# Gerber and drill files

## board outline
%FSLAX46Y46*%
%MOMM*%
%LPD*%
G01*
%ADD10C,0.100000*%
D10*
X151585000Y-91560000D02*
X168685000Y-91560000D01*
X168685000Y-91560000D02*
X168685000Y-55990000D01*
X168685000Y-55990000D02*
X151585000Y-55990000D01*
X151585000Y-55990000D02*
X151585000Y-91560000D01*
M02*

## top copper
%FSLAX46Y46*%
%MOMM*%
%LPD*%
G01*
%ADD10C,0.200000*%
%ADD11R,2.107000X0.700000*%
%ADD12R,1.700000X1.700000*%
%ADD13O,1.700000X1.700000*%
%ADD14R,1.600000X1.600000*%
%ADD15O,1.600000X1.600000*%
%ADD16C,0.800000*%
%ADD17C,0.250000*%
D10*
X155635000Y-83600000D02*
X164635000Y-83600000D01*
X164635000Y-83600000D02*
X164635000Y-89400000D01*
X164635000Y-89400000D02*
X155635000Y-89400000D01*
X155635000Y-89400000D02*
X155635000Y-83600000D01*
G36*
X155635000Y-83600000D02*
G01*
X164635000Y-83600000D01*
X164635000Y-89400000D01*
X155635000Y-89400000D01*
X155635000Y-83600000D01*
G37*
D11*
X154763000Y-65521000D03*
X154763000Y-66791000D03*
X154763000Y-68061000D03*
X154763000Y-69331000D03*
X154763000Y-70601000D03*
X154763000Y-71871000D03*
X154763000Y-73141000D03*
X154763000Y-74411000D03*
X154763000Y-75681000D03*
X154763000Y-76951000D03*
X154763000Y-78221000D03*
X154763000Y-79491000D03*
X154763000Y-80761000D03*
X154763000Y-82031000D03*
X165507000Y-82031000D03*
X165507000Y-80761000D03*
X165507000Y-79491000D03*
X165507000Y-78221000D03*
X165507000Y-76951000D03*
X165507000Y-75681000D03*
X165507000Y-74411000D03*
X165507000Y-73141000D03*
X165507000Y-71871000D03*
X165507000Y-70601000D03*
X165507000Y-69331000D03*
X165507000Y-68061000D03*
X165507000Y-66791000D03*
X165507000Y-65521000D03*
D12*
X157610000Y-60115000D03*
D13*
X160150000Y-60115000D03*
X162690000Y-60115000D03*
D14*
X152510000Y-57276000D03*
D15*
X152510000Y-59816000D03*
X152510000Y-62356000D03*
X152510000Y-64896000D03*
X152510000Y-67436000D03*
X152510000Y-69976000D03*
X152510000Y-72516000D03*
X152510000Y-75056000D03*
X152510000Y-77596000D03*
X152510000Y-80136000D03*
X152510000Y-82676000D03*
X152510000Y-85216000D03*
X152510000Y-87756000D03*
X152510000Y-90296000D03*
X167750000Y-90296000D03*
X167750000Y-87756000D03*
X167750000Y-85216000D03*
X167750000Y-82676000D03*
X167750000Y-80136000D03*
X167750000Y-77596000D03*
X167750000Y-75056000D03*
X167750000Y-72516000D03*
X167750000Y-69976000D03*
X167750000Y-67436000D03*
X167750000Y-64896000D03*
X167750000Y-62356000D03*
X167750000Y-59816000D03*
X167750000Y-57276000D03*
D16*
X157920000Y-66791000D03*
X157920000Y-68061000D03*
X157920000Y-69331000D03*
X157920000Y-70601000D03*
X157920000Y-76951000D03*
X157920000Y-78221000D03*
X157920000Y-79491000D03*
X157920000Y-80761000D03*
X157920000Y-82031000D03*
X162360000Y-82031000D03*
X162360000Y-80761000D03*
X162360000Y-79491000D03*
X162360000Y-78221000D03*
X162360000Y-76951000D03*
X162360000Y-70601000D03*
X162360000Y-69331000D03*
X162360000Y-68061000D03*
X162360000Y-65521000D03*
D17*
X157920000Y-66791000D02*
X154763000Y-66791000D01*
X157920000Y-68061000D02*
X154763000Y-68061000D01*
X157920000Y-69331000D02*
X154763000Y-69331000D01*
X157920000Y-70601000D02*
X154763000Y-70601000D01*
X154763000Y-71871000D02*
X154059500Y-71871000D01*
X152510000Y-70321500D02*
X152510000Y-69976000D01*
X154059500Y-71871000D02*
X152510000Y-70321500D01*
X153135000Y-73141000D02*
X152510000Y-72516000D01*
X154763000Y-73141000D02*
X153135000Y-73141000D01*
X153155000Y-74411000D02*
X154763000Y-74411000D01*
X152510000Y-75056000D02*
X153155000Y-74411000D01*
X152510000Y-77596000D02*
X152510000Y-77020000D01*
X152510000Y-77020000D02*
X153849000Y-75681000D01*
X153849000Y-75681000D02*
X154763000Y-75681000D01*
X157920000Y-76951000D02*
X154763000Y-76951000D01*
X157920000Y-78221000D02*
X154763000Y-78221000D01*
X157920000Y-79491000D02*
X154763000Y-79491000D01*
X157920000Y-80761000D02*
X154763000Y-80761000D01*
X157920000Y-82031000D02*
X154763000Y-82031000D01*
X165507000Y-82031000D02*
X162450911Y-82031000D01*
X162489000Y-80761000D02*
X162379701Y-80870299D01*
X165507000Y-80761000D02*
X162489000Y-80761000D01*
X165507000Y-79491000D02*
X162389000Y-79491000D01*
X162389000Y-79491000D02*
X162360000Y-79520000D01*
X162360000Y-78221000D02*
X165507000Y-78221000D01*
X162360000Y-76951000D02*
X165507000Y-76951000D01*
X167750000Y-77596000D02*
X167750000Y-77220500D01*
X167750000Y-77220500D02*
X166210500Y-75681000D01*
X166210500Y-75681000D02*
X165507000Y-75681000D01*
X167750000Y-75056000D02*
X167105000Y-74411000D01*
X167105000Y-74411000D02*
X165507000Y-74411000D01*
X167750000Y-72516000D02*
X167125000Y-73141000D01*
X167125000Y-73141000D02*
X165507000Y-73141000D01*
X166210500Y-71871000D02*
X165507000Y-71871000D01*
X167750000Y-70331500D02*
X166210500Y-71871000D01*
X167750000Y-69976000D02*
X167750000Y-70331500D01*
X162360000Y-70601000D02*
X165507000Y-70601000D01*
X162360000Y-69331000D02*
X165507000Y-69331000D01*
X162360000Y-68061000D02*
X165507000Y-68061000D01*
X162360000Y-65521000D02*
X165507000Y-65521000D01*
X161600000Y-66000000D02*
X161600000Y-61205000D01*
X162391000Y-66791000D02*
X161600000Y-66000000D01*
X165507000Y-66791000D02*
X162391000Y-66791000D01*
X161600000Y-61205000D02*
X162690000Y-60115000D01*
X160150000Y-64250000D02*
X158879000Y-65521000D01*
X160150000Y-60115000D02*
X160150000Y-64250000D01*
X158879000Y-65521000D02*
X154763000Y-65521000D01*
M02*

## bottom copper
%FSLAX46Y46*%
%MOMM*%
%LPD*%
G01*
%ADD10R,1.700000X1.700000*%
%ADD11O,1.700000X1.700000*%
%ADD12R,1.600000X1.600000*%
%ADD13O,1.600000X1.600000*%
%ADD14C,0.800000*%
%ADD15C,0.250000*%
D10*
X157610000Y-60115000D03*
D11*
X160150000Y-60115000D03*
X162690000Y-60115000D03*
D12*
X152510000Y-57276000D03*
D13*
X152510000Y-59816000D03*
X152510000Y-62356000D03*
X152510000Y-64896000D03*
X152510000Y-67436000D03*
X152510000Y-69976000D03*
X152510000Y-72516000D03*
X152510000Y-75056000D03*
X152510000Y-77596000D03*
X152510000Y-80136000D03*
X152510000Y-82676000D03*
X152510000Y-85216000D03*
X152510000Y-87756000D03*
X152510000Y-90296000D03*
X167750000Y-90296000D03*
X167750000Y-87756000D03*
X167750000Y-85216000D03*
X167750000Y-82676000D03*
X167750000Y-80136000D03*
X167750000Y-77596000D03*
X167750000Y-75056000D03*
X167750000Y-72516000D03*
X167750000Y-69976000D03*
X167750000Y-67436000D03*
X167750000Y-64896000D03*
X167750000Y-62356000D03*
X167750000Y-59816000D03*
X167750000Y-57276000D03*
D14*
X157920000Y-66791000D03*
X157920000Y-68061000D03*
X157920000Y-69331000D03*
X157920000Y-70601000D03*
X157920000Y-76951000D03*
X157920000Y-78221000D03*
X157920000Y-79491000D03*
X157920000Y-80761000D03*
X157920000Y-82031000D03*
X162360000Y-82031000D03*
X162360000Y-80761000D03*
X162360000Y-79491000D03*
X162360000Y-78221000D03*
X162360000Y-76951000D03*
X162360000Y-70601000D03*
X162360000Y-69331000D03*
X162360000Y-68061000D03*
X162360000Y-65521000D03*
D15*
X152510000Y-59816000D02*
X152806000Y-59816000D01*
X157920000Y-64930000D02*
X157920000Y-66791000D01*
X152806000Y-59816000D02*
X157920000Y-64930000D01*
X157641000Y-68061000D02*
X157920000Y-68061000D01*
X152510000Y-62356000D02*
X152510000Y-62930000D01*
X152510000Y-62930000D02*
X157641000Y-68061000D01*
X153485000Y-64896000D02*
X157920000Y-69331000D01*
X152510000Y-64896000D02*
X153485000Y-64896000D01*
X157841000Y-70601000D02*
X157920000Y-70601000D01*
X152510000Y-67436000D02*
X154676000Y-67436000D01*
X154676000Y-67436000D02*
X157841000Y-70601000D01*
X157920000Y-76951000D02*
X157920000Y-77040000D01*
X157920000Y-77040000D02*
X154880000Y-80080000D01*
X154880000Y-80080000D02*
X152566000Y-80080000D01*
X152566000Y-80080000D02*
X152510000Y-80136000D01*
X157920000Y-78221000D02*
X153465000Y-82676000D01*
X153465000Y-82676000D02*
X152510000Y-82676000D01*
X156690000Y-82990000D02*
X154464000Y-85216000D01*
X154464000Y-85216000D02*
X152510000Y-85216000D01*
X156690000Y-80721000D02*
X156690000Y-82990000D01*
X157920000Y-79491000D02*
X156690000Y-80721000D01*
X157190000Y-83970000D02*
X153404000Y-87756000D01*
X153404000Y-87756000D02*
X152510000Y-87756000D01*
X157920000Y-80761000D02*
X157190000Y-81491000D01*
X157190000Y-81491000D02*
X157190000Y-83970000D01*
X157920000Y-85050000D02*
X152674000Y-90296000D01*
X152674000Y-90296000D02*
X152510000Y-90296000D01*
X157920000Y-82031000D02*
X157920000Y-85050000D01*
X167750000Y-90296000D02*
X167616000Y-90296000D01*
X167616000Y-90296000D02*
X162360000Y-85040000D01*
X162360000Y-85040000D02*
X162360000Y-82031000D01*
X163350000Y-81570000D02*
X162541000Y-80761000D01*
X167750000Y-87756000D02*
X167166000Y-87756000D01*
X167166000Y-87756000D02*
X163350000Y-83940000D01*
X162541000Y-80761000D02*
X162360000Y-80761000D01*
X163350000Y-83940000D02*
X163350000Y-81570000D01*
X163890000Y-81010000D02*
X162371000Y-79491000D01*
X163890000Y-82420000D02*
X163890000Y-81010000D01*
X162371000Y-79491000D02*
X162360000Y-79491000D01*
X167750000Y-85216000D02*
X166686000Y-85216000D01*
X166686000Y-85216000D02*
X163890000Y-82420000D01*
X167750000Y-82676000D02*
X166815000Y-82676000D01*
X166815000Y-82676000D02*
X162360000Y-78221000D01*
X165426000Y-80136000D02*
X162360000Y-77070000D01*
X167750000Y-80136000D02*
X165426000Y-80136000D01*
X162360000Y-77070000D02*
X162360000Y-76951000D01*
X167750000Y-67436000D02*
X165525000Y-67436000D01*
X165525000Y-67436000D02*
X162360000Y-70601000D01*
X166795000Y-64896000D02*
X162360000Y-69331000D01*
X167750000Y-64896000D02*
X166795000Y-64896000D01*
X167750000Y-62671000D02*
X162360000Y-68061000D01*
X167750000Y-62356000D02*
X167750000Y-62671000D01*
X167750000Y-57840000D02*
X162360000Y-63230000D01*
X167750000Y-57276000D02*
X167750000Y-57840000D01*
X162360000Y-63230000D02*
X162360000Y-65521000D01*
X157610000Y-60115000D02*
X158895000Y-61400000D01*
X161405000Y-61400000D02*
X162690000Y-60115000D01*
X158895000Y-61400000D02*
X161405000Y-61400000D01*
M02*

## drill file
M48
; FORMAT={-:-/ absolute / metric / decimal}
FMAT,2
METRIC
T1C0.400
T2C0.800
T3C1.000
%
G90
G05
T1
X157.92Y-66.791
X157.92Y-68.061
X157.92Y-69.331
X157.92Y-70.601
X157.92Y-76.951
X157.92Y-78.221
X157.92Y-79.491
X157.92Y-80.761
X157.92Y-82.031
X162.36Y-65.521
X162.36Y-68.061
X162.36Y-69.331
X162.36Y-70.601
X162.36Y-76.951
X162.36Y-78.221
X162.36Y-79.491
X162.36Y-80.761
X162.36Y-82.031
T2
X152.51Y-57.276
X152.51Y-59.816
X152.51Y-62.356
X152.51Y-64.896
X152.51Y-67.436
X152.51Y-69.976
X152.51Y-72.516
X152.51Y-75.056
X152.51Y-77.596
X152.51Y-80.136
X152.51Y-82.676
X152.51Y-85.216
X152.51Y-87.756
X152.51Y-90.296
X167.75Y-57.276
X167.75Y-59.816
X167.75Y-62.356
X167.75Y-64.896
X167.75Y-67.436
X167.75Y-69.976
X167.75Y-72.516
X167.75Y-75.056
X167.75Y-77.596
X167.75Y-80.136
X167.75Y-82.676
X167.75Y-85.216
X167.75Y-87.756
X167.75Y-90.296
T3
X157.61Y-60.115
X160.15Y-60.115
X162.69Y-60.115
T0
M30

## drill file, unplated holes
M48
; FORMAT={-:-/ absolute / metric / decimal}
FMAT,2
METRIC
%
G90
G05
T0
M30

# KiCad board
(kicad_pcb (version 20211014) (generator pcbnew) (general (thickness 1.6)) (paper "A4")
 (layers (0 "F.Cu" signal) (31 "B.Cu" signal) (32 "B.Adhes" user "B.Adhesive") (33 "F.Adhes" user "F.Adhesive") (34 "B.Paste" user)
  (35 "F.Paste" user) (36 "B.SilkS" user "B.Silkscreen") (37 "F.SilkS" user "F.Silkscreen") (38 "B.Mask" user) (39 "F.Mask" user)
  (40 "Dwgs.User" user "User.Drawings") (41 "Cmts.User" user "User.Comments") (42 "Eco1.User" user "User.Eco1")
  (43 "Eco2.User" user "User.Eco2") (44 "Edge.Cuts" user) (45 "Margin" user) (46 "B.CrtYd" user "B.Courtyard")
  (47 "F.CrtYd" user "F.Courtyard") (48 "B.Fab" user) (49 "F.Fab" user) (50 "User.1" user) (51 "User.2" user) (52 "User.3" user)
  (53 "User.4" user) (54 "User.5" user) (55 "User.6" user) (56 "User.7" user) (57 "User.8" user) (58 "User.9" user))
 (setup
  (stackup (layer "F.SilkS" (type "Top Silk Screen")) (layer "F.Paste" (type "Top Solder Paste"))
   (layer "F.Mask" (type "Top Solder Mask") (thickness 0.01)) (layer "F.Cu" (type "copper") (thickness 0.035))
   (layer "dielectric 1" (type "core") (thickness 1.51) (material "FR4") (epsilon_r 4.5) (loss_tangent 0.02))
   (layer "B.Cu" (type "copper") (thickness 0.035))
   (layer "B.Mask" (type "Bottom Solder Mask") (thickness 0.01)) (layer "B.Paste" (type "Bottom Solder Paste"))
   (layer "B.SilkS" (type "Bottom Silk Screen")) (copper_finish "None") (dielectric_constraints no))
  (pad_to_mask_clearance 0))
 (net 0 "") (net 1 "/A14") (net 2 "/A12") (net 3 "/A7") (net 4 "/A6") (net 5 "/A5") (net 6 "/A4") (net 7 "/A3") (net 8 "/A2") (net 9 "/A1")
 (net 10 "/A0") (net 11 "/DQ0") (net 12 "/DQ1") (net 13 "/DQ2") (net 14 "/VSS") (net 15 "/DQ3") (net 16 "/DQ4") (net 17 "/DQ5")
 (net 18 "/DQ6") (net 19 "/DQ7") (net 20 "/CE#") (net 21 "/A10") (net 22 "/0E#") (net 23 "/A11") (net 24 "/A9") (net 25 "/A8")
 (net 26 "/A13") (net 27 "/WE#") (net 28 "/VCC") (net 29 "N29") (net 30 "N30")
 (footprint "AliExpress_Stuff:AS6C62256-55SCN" (layer "F.Cu") (at 160.135 73.776)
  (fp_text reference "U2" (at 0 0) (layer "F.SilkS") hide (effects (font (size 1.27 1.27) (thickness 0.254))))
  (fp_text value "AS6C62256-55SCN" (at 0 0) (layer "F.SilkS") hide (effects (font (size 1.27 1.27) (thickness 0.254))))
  (pad "1" smd rect (at -5.372 -8.255 90) (size 0.7 2.107) (layers "F.Cu" "F.Paste" "F.Mask") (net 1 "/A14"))
  (pad "2" smd rect (at -5.372 -6.985 90) (size 0.7 2.107) (layers "F.Cu" "F.Paste" "F.Mask") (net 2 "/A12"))
  (pad "3" smd rect (at -5.372 -5.715 90) (size 0.7 2.107) (layers "F.Cu" "F.Paste" "F.Mask") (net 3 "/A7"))
  (pad "4" smd rect (at -5.372 -4.445 90) (size 0.7 2.107) (layers "F.Cu" "F.Paste" "F.Mask") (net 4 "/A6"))
  (pad "5" smd rect (at -5.372 -3.175 90) (size 0.7 2.107) (layers "F.Cu" "F.Paste" "F.Mask") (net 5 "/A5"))
  (pad "6" smd rect (at -5.372 -1.905 90) (size 0.7 2.107) (layers "F.Cu" "F.Paste" "F.Mask") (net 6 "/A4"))
  (pad "7" smd rect (at -5.372 -0.635 90) (size 0.7 2.107) (layers "F.Cu" "F.Paste" "F.Mask") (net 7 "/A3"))
  (pad "8" smd rect (at -5.372 0.635 90) (size 0.7 2.107) (layers "F.Cu" "F.Paste" "F.Mask") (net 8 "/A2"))
  (pad "9" smd rect (at -5.372 1.905 90) (size 0.7 2.107) (layers "F.Cu" "F.Paste" "F.Mask") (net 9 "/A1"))
  (pad "10" smd rect (at -5.372 3.175 90) (size 0.7 2.107) (layers "F.Cu" "F.Paste" "F.Mask") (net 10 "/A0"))
  (pad "11" smd rect (at -5.372 4.445 90) (size 0.7 2.107) (layers "F.Cu" "F.Paste" "F.Mask") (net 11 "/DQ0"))
  (pad "12" smd rect (at -5.372 5.715 90) (size 0.7 2.107) (layers "F.Cu" "F.Paste" "F.Mask") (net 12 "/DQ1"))
  (pad "13" smd rect (at -5.372 6.985 90) (size 0.7 2.107) (layers "F.Cu" "F.Paste" "F.Mask") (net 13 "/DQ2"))
  (pad "14" smd rect (at -5.372 8.255 90) (size 0.7 2.107) (layers "F.Cu" "F.Paste" "F.Mask") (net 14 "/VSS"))
  (pad "15" smd rect (at 5.372 8.255 90) (size 0.7 2.107) (layers "F.Cu" "F.Paste" "F.Mask") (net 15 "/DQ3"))
  (pad "16" smd rect (at 5.372 6.985 90) (size 0.7 2.107) (layers "F.Cu" "F.Paste" "F.Mask") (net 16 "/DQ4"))
  (pad "17" smd rect (at 5.372 5.715 90) (size 0.7 2.107) (layers "F.Cu" "F.Paste" "F.Mask") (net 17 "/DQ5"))
  (pad "18" smd rect (at 5.372 4.445 90) (size 0.7 2.107) (layers "F.Cu" "F.Paste" "F.Mask") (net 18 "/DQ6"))
  (pad "19" smd rect (at 5.372 3.175 90) (size 0.7 2.107) (layers "F.Cu" "F.Paste" "F.Mask") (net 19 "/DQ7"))
  (pad "20" smd rect (at 5.372 1.905 90) (size 0.7 2.107) (layers "F.Cu" "F.Paste" "F.Mask") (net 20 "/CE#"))
  (pad "21" smd rect (at 5.372 0.635 90) (size 0.7 2.107) (layers "F.Cu" "F.Paste" "F.Mask") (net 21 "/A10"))
  (pad "22" smd rect (at 5.372 -0.635 90) (size 0.7 2.107) (layers "F.Cu" "F.Paste" "F.Mask") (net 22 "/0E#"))
  (pad "23" smd rect (at 5.372 -1.905 90) (size 0.7 2.107) (layers "F.Cu" "F.Paste" "F.Mask") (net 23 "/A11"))
  (pad "24" smd rect (at 5.372 -3.175 90) (size 0.7 2.107) (layers "F.Cu" "F.Paste" "F.Mask") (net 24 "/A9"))
  (pad "25" smd rect (at 5.372 -4.445 90) (size 0.7 2.107) (layers "F.Cu" "F.Paste" "F.Mask") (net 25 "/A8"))
  (pad "26" smd rect (at 5.372 -5.715 90) (size 0.7 2.107) (layers "F.Cu" "F.Paste" "F.Mask") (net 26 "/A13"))
  (pad "27" smd rect (at 5.372 -6.985 90) (size 0.7 2.107) (layers "F.Cu" "F.Paste" "F.Mask") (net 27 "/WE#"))
  (pad "28" smd rect (at 5.372 -8.255 90) (size 0.7 2.107) (layers "F.Cu" "F.Paste" "F.Mask") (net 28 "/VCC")))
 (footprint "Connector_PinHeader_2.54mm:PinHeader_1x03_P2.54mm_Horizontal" (layer "F.Cu") (at 157.61 60.115 90)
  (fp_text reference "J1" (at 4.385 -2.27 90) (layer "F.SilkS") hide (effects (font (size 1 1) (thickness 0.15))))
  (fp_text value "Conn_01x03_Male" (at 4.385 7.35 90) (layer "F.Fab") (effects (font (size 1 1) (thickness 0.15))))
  (pad "1" thru_hole rect (at 0 0 90) (size 1.7 1.7) (drill 1) (layers *.Cu *.Mask) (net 27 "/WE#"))
  (pad "2" thru_hole oval (at 0 2.54 90) (size 1.7 1.7) (drill 1) (layers *.Cu *.Mask) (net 1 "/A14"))
  (pad "3" thru_hole oval (at 0 5.08 90) (size 1.7 1.7) (drill 1) (layers *.Cu *.Mask) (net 27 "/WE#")))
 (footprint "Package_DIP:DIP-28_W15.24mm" (layer "F.Cu") (at 152.51 57.276)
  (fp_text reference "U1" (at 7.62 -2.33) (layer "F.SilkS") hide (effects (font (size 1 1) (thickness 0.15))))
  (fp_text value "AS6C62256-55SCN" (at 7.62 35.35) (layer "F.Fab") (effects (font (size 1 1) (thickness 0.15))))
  (pad "1" thru_hole rect (at 0 0) (size 1.6 1.6) (drill 0.8) (layers *.Cu *.Mask) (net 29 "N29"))
  (pad "2" thru_hole oval (at 0 2.54) (size 1.6 1.6) (drill 0.8) (layers *.Cu *.Mask) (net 2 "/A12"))
  (pad "3" thru_hole oval (at 0 5.08) (size 1.6 1.6) (drill 0.8) (layers *.Cu *.Mask) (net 3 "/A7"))
  (pad "4" thru_hole oval (at 0 7.62) (size 1.6 1.6) (drill 0.8) (layers *.Cu *.Mask) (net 4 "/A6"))
  (pad "5" thru_hole oval (at 0 10.16) (size 1.6 1.6) (drill 0.8) (layers *.Cu *.Mask) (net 5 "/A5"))
  (pad "6" thru_hole oval (at 0 12.7) (size 1.6 1.6) (drill 0.8) (layers *.Cu *.Mask) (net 6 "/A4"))
  (pad "7" thru_hole oval (at 0 15.24) (size 1.6 1.6) (drill 0.8) (layers *.Cu *.Mask) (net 7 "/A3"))
  (pad "8" thru_hole oval (at 0 17.78) (size 1.6 1.6) (drill 0.8) (layers *.Cu *.Mask) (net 8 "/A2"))
  (pad "9" thru_hole oval (at 0 20.32) (size 1.6 1.6) (drill 0.8) (layers *.Cu *.Mask) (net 9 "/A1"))
  (pad "10" thru_hole oval (at 0 22.86) (size 1.6 1.6) (drill 0.8) (layers *.Cu *.Mask) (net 10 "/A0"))
  (pad "11" thru_hole oval (at 0 25.4) (size 1.6 1.6) (drill 0.8) (layers *.Cu *.Mask) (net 11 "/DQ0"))
  (pad "12" thru_hole oval (at 0 27.94) (size 1.6 1.6) (drill 0.8) (layers *.Cu *.Mask) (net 12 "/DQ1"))
  (pad "13" thru_hole oval (at 0 30.48) (size 1.6 1.6) (drill 0.8) (layers *.Cu *.Mask) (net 13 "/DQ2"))
  (pad "14" thru_hole oval (at 0 33.02) (size 1.6 1.6) (drill 0.8) (layers *.Cu *.Mask) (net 14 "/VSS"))
  (pad "15" thru_hole oval (at 15.24 33.02) (size 1.6 1.6) (drill 0.8) (layers *.Cu *.Mask) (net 15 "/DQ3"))
  (pad "16" thru_hole oval (at 15.24 30.48) (size 1.6 1.6) (drill 0.8) (layers *.Cu *.Mask) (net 16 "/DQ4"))
  (pad "17" thru_hole oval (at 15.24 27.94) (size 1.6 1.6) (drill 0.8) (layers *.Cu *.Mask) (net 17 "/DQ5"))
  (pad "18" thru_hole oval (at 15.24 25.4) (size 1.6 1.6) (drill 0.8) (layers *.Cu *.Mask) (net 18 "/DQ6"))
  (pad "19" thru_hole oval (at 15.24 22.86) (size 1.6 1.6) (drill 0.8) (layers *.Cu *.Mask) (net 19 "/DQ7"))
  (pad "20" thru_hole oval (at 15.24 20.32) (size 1.6 1.6) (drill 0.8) (layers *.Cu *.Mask) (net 20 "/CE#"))
  (pad "21" thru_hole oval (at 15.24 17.78) (size 1.6 1.6) (drill 0.8) (layers *.Cu *.Mask) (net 21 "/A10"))
  (pad "22" thru_hole oval (at 15.24 15.24) (size 1.6 1.6) (drill 0.8) (layers *.Cu *.Mask) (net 22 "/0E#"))
  (pad "23" thru_hole oval (at 15.24 12.7) (size 1.6 1.6) (drill 0.8) (layers *.Cu *.Mask) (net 23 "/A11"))
  (pad "24" thru_hole oval (at 15.24 10.16) (size 1.6 1.6) (drill 0.8) (layers *.Cu *.Mask) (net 24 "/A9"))
  (pad "25" thru_hole oval (at 15.24 7.62) (size 1.6 1.6) (drill 0.8) (layers *.Cu *.Mask) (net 25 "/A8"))
  (pad "26" thru_hole oval (at 15.24 5.08) (size 1.6 1.6) (drill 0.8) (layers *.Cu *.Mask) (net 26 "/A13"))
  (pad "27" thru_hole oval (at 15.24 2.54) (size 1.6 1.6) (drill 0.8) (layers *.Cu *.Mask) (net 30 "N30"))
  (pad "28" thru_hole oval (at 15.24 0) (size 1.6 1.6) (drill 0.8) (layers *.Cu *.Mask) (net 28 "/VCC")))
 (gr_rect (start 155.635 83.6) (end 164.635 89.4) (layer "F.Cu") (width 0.2) (fill solid))
 (gr_rect (start 151.585 91.56) (end 168.685 55.99) (layer "Edge.Cuts") (width 0.1) (fill none))
 (segment (start 157.92 66.791) (end 154.763 66.791) (width 0.25) (layer "F.Cu") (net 2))
 (via (at 157.92 66.791) (size 0.8) (drill 0.4) (layers "F.Cu" "B.Cu") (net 2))
 (segment (start 152.51 59.816) (end 152.806 59.816) (width 0.25) (layer "B.Cu") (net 2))
 (segment (start 157.92 64.93) (end 157.92 66.791) (width 0.25) (layer "B.Cu") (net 2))
 (segment (start 152.806 59.816) (end 157.92 64.93) (width 0.25) (layer "B.Cu") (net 2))
 (segment (start 157.92 68.061) (end 154.763 68.061) (width 0.25) (layer "F.Cu") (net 3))
 (via (at 157.92 68.061) (size 0.8) (drill 0.4) (layers "F.Cu" "B.Cu") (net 3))
 (segment (start 157.641 68.061) (end 157.92 68.061) (width 0.25) (layer "B.Cu") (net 3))
 (segment (start 152.51 62.356) (end 152.51 62.93) (width 0.25) (layer "B.Cu") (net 3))
 (segment (start 152.51 62.93) (end 157.641 68.061) (width 0.25) (layer "B.Cu") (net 3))
 (segment (start 157.92 69.331) (end 154.763 69.331) (width 0.25) (layer "F.Cu") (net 4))
 (via (at 157.92 69.331) (size 0.8) (drill 0.4) (layers "F.Cu" "B.Cu") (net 4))
 (segment (start 153.485 64.896) (end 157.92 69.331) (width 0.25) (layer "B.Cu") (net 4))
 (segment (start 152.51 64.896) (end 153.485 64.896) (width 0.25) (layer "B.Cu") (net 4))
 (segment (start 157.92 70.601) (end 154.763 70.601) (width 0.25) (layer "F.Cu") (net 5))
 (via (at 157.92 70.601) (size 0.8) (drill 0.4) (layers "F.Cu" "B.Cu") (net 5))
 (segment (start 157.841 70.601) (end 157.92 70.601) (width 0.25) (layer "B.Cu") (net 5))
 (segment (start 152.51 67.436) (end 154.676 67.436) (width 0.25) (layer "B.Cu") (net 5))
 (segment (start 154.676 67.436) (end 157.841 70.601) (width 0.25) (layer "B.Cu") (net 5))
 (segment (start 154.763 71.871) (end 154.0595 71.871) (width 0.25) (layer "F.Cu") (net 6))
 (segment (start 152.51 70.3215) (end 152.51 69.976) (width 0.25) (layer "F.Cu") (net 6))
 (segment (start 154.0595 71.871) (end 152.51 70.3215) (width 0.25) (layer "F.Cu") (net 6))
 (segment (start 153.135 73.141) (end 152.51 72.516) (width 0.25) (layer "F.Cu") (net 7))
 (segment (start 154.763 73.141) (end 153.135 73.141) (width 0.25) (layer "F.Cu") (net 7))
 (segment (start 153.155 74.411) (end 154.763 74.411) (width 0.25) (layer "F.Cu") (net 8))
 (segment (start 152.51 75.056) (end 153.155 74.411) (width 0.25) (layer "F.Cu") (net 8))
 (segment (start 152.51 77.596) (end 152.51 77.02) (width 0.25) (layer "F.Cu") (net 9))
 (segment (start 152.51 77.02) (end 153.849 75.681) (width 0.25) (layer "F.Cu") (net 9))
 (segment (start 153.849 75.681) (end 154.763 75.681) (width 0.25) (layer "F.Cu") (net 9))
 (segment (start 157.92 76.951) (end 154.763 76.951) (width 0.25) (layer "F.Cu") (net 10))
 (via (at 157.92 76.951) (size 0.8) (drill 0.4) (layers "F.Cu" "B.Cu") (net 10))
 (segment (start 157.92 76.951) (end 157.92 77.04) (width 0.25) (layer "B.Cu") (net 10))
 (segment (start 157.92 77.04) (end 154.88 80.08) (width 0.25) (layer "B.Cu") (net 10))
 (segment (start 154.88 80.08) (end 152.566 80.08) (width 0.25) (layer "B.Cu") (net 10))
 (segment (start 152.566 80.08) (end 152.51 80.136) (width 0.25) (layer "B.Cu") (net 10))
 (segment (start 157.92 78.221) (end 154.763 78.221) (width 0.25) (layer "F.Cu") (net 11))
 (via (at 157.92 78.221) (size 0.8) (drill 0.4) (layers "F.Cu" "B.Cu") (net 11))
 (segment (start 157.92 78.221) (end 153.465 82.676) (width 0.25) (layer "B.Cu") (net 11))
 (segment (start 153.465 82.676) (end 152.51 82.676) (width 0.25) (layer "B.Cu") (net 11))
 (segment (start 157.92 79.491) (end 154.763 79.491) (width 0.25) (layer "F.Cu") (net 12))
 (via (at 157.92 79.491) (size 0.8) (drill 0.4) (layers "F.Cu" "B.Cu") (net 12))
 (segment (start 156.69 82.99) (end 154.464 85.216) (width 0.25) (layer "B.Cu") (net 12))
 (segment (start 154.464 85.216) (end 152.51 85.216) (width 0.25) (layer "B.Cu") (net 12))
 (segment (start 156.69 80.721) (end 156.69 82.99) (width 0.25) (layer "B.Cu") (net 12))
 (segment (start 157.92 79.491) (end 156.69 80.721) (width 0.25) (layer "B.Cu") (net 12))
 (segment (start 157.92 80.761) (end 154.763 80.761) (width 0.25) (layer "F.Cu") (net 13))
 (via (at 157.92 80.761) (size 0.8) (drill 0.4) (layers "F.Cu" "B.Cu") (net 13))
 (segment (start 157.19 83.97) (end 153.404 87.756) (width 0.25) (layer "B.Cu") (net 13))
 (segment (start 153.404 87.756) (end 152.51 87.756) (width 0.25) (layer "B.Cu") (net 13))
 (segment (start 157.92 80.761) (end 157.19 81.491) (width 0.25) (layer "B.Cu") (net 13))
 (segment (start 157.19 81.491) (end 157.19 83.97) (width 0.25) (layer "B.Cu") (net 13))
 (segment (start 157.92 82.031) (end 154.763 82.031) (width 0.25) (layer "F.Cu") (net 14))
 (via (at 157.92 82.031) (size 0.8) (drill 0.4) (layers "F.Cu" "B.Cu") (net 14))
 (segment (start 157.92 85.05) (end 152.674 90.296) (width 0.25) (layer "B.Cu") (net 14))
 (segment (start 152.674 90.296) (end 152.51 90.296) (width 0.25) (layer "B.Cu") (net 14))
 (segment (start 157.92 82.031) (end 157.92 85.05) (width 0.25) (layer "B.Cu") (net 14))
 (segment (start 165.507 82.031) (end 162.450911 82.031) (width 0.25) (layer "F.Cu") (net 15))
 (via (at 162.36 82.031) (size 0.8) (drill 0.4) (layers "F.Cu" "B.Cu") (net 15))
 (segment (start 167.75 90.296) (end 167.616 90.296) (width 0.25) (layer "B.Cu") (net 15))
 (segment (start 167.616 90.296) (end 162.36 85.04) (width 0.25) (layer "B.Cu") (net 15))
 (segment (start 162.36 85.04) (end 162.36 82.031) (width 0.25) (layer "B.Cu") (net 15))
 (segment (start 162.489 80.761) (end 162.379701 80.870299) (width 0.25) (layer "F.Cu") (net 16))
 (segment (start 165.507 80.761) (end 162.489 80.761) (width 0.25) (layer "F.Cu") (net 16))
 (via (at 162.36 80.761) (size 0.8) (drill 0.4) (layers "F.Cu" "B.Cu") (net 16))
 (segment (start 163.35 81.57) (end 162.541 80.761) (width 0.25) (layer "B.Cu") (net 16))
 (segment (start 167.75 87.756) (end 167.166 87.756) (width 0.25) (layer "B.Cu") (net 16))
 (segment (start 167.166 87.756) (end 163.35 83.94) (width 0.25) (layer "B.Cu") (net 16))
 (segment (start 162.541 80.761) (end 162.36 80.761) (width 0.25) (layer "B.Cu") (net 16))
 (segment (start 163.35 83.94) (end 163.35 81.57) (width 0.25) (layer "B.Cu") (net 16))
 (segment (start 165.507 79.491) (end 162.389 79.491) (width 0.25) (layer "F.Cu") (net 17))
 (segment (start 162.389 79.491) (end 162.36 79.52) (width 0.25) (layer "F.Cu") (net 17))
 (via (at 162.36 79.491) (size 0.8) (drill 0.4) (layers "F.Cu" "B.Cu") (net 17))
 (segment (start 163.89 81.01) (end 162.371 79.491) (width 0.25) (layer "B.Cu") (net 17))
 (segment (start 163.89 82.42) (end 163.89 81.01) (width 0.25) (layer "B.Cu") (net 17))
 (segment (start 162.371 79.491) (end 162.36 79.491) (width 0.25) (layer "B.Cu") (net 17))
 (segment (start 167.75 85.216) (end 166.686 85.216) (width 0.25) (layer "B.Cu") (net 17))
 (segment (start 166.686 85.216) (end 163.89 82.42) (width 0.25) (layer "B.Cu") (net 17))
 (segment (start 162.36 78.221) (end 165.507 78.221) (width 0.25) (layer "F.Cu") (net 18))
 (via (at 162.36 78.221) (size 0.8) (drill 0.4) (layers "F.Cu" "B.Cu") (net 18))
 (segment (start 167.75 82.676) (end 166.815 82.676) (width 0.25) (layer "B.Cu") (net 18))
 (segment (start 166.815 82.676) (end 162.36 78.221) (width 0.25) (layer "B.Cu") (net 18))
 (segment (start 162.36 76.951) (end 165.507 76.951) (width 0.25) (layer "F.Cu") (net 19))
 (via (at 162.36 76.951) (size 0.8) (drill 0.4) (layers "F.Cu" "B.Cu") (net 19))
 (segment (start 165.426 80.136) (end 162.36 77.07) (width 0.25) (layer "B.Cu") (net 19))
 (segment (start 167.75 80.136) (end 165.426 80.136) (width 0.25) (layer "B.Cu") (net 19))
 (segment (start 162.36 77.07) (end 162.36 76.951) (width 0.25) (layer "B.Cu") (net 19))
 (segment (start 167.75 77.596) (end 167.75 77.2205) (width 0.25) (layer "F.Cu") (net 20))
 (segment (start 167.75 77.2205) (end 166.2105 75.681) (width 0.25) (layer "F.Cu") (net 20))
 (segment (start 166.2105 75.681) (end 165.507 75.681) (width 0.25) (layer "F.Cu") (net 20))
 (segment (start 167.75 75.056) (end 167.105 74.411) (width 0.25) (layer "F.Cu") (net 21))
 (segment (start 167.105 74.411) (end 165.507 74.411) (width 0.25) (layer "F.Cu") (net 21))
 (segment (start 167.75 72.516) (end 167.125 73.141) (width 0.25) (layer "F.Cu") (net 22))
 (segment (start 167.125 73.141) (end 165.507 73.141) (width 0.25) (layer "F.Cu") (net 22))
 (segment (start 166.2105 71.871) (end 165.507 71.871) (width 0.25) (layer "F.Cu") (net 23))
 (segment (start 167.75 70.3315) (end 166.2105 71.871) (width 0.25) (layer "F.Cu") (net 23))
 (segment (start 167.75 69.976) (end 167.75 70.3315) (width 0.25) (layer "F.Cu") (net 23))
 (segment (start 162.36 70.601) (end 165.507 70.601) (width 0.25) (layer "F.Cu") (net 24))
 (via (at 162.36 70.601) (size 0.8) (drill 0.4) (layers "F.Cu" "B.Cu") (free) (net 24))
 (segment (start 167.75 67.436) (end 165.525 67.436) (width 0.25) (layer "B.Cu") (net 24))
 (segment (start 165.525 67.436) (end 162.36 70.601) (width 0.25) (layer "B.Cu") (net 24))
 (segment (start 162.36 69.331) (end 165.507 69.331) (width 0.25) (layer "F.Cu") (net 25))
 (via (at 162.36 69.331) (size 0.8) (drill 0.4) (layers "F.Cu" "B.Cu") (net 25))
 (segment (start 166.795 64.896) (end 162.36 69.331) (width 0.25) (layer "B.Cu") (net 25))
 (segment (start 167.75 64.896) (end 166.795 64.896) (width 0.25) (layer "B.Cu") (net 25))
 (segment (start 162.36 68.061) (end 165.507 68.061) (width 0.25) (layer "F.Cu") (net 26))
 (via (at 162.36 68.061) (size 0.8) (drill 0.4) (layers "F.Cu" "B.Cu") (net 26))
 (segment (start 167.75 62.671) (end 162.36 68.061) (width 0.25) (layer "B.Cu") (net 26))
 (segment (start 167.75 62.356) (end 167.75 62.671) (width 0.25) (layer "B.Cu") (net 26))
 (segment (start 162.36 65.521) (end 165.507 65.521) (width 0.25) (layer "F.Cu") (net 28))
 (via (at 162.36 65.521) (size 0.8) (drill 0.4) (layers "F.Cu" "B.Cu") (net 28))
 (segment (start 167.75 57.84) (end 162.36 63.23) (width 0.25) (layer "B.Cu") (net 28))
 (segment (start 167.75 57.276) (end 167.75 57.84) (width 0.25) (layer "B.Cu") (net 28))
 (segment (start 162.36 63.23) (end 162.36 65.521) (width 0.25) (layer "B.Cu") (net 28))
 (segment (start 161.6 66) (end 161.6 61.205) (width 0.25) (layer "F.Cu") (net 27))
 (segment (start 162.391 66.791) (end 161.6 66) (width 0.25) (layer "F.Cu") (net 27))
 (segment (start 165.507 66.791) (end 162.391 66.791) (width 0.25) (layer "F.Cu") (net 27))
 (segment (start 161.6 61.205) (end 162.69 60.115) (width 0.25) (layer "F.Cu") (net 27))
 (segment (start 157.61 60.115) (end 158.895 61.4) (width 0.25) (layer "B.Cu") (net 27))
 (segment (start 161.405 61.4) (end 162.69 60.115) (width 0.25) (layer "B.Cu") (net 27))
 (segment (start 158.895 61.4) (end 161.405 61.4) (width 0.25) (layer "B.Cu") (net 27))
 (segment (start 160.15 64.25) (end 158.879 65.521) (width 0.25) (layer "F.Cu") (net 1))
 (segment (start 160.15 60.115) (end 160.15 64.25) (width 0.25) (layer "F.Cu") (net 1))
 (segment (start 158.879 65.521) (end 154.763 65.521) (width 0.25) (layer "F.Cu") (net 1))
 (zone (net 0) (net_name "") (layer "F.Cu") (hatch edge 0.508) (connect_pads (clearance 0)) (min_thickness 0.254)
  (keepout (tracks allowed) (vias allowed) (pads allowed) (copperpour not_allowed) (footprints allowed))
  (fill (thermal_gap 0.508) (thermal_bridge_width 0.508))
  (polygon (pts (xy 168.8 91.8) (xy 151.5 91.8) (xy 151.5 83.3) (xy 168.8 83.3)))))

